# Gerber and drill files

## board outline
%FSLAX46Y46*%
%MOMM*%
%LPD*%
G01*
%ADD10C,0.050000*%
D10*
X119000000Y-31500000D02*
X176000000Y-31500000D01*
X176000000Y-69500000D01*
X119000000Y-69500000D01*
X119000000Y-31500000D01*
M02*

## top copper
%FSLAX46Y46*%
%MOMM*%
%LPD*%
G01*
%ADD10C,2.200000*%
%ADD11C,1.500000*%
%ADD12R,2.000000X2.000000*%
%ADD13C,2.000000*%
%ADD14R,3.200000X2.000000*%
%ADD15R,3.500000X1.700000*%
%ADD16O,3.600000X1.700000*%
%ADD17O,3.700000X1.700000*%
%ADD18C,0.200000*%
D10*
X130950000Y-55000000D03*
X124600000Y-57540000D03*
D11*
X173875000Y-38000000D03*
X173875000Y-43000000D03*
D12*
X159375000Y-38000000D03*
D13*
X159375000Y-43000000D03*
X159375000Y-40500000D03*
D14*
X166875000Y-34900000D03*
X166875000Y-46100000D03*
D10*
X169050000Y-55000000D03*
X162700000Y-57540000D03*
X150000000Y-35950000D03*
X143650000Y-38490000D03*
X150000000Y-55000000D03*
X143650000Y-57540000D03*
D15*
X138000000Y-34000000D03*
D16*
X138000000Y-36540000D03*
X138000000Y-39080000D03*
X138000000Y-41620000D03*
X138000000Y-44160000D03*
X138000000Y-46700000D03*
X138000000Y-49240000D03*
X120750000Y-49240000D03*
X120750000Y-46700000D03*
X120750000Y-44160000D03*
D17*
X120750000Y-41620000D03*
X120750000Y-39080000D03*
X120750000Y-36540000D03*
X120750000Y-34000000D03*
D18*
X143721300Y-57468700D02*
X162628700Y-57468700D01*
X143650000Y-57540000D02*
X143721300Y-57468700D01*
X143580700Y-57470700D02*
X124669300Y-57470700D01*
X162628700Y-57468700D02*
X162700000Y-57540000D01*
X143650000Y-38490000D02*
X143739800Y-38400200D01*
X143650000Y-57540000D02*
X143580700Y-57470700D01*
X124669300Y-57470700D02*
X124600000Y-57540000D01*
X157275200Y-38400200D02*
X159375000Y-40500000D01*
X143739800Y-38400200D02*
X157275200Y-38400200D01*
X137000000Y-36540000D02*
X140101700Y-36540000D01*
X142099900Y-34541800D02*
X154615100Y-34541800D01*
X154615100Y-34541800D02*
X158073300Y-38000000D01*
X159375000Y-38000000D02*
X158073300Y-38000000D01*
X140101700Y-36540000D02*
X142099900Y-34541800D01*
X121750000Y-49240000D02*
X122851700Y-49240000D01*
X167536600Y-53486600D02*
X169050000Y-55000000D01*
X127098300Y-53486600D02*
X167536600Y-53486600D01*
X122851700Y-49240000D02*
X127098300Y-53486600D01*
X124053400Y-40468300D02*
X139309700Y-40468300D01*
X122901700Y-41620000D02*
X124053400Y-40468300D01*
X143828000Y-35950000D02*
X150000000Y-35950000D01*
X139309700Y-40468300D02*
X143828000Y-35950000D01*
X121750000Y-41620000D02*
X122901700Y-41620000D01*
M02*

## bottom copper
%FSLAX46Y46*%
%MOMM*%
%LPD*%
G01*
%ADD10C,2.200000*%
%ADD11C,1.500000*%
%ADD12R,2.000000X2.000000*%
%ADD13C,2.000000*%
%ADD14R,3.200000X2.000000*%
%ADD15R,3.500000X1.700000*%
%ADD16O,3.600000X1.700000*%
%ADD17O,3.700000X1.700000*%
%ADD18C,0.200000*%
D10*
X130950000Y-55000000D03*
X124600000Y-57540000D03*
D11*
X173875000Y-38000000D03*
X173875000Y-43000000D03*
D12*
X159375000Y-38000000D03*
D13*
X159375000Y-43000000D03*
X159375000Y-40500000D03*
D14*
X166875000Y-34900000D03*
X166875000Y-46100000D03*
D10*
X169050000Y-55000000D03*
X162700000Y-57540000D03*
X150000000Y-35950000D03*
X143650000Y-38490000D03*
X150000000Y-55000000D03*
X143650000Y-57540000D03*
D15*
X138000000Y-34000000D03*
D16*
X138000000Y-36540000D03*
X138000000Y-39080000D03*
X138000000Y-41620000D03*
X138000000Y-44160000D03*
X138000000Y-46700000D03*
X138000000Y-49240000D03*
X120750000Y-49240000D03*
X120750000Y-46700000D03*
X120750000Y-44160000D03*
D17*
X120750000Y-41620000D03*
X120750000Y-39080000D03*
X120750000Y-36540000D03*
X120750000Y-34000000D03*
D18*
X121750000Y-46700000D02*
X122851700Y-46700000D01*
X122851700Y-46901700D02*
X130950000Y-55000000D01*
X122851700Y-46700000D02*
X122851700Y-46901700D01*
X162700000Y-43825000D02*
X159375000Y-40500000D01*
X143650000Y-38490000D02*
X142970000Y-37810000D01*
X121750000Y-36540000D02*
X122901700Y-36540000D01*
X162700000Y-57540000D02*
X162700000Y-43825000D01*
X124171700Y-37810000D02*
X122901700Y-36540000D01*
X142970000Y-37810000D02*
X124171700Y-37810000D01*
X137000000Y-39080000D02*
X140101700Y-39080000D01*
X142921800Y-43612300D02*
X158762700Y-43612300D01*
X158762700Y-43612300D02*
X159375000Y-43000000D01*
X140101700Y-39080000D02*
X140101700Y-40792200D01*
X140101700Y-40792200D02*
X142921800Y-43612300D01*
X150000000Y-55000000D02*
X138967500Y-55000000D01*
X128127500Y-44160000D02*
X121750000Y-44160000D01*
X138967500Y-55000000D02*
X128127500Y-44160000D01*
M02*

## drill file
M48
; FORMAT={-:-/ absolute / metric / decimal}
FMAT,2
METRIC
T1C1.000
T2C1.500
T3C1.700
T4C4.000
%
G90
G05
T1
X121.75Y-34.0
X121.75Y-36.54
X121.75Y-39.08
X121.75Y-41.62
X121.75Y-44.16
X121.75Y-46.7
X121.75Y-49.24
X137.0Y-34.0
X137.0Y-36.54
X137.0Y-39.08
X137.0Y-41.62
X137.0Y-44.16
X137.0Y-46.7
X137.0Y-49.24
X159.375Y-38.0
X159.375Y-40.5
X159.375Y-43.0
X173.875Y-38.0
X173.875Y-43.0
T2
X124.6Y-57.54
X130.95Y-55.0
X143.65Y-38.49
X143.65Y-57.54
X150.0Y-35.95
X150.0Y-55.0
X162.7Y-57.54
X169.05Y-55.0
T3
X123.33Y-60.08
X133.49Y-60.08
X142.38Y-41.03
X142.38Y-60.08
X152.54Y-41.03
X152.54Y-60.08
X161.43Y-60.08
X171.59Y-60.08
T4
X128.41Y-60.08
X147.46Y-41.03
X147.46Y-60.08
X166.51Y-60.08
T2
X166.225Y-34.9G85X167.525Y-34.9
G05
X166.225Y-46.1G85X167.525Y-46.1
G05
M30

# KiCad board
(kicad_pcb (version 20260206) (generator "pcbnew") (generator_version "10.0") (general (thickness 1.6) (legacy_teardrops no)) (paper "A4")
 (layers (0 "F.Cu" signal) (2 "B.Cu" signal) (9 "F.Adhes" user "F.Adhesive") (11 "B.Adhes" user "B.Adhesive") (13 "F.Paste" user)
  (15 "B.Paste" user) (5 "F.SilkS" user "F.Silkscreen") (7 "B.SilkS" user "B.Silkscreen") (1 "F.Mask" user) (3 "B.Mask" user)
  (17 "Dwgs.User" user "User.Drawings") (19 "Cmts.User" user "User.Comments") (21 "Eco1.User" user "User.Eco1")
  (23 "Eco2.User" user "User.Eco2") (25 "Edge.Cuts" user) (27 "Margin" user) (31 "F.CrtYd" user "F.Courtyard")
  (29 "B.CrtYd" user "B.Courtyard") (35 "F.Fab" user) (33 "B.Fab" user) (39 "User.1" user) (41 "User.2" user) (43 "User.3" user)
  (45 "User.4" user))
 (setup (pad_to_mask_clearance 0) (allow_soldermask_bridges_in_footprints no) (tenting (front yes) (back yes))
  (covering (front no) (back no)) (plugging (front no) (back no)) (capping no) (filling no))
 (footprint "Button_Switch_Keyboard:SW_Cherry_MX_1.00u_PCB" (layer "F.Cu") (at 130.95 55)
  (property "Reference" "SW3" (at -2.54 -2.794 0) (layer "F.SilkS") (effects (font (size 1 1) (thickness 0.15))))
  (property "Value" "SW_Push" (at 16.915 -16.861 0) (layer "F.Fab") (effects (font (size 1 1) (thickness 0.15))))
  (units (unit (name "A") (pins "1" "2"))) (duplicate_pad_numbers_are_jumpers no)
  (pad "" np_thru_hole circle (at -7.62 5.08) (size 1.7 1.7) (drill 1.7) (layers "*.Cu" "*.Mask"))
  (pad "" np_thru_hole circle (at -2.54 5.08) (size 4 4) (drill 4) (layers "*.Cu" "*.Mask"))
  (pad "" np_thru_hole circle (at 2.54 5.08) (size 1.7 1.7) (drill 1.7) (layers "*.Cu" "*.Mask"))
  (pad "1" thru_hole circle (at 0 0) (size 2.2 2.2) (drill 1.5) (layers "*.Cu" "*.Mask") (remove_unused_layers no)
   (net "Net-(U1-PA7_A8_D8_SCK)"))
  (pad "2" thru_hole circle (at -6.35 2.54) (size 2.2 2.2) (drill 1.5) (layers "*.Cu" "*.Mask") (remove_unused_layers no) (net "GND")))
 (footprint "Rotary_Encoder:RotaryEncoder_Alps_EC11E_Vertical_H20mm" (layer "F.Cu") (at 159.375 38)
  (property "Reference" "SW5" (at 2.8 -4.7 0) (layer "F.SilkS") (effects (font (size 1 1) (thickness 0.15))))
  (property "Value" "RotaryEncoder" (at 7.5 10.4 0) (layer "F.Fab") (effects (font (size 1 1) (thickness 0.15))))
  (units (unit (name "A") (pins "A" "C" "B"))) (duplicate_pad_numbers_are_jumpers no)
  (pad "" thru_hole circle (at 14.5 0) (size 1.5 1.5) (drill 1) (layers "*.Cu" "*.Mask") (remove_unused_layers no))
  (pad "" thru_hole circle (at 14.5 5) (size 1.5 1.5) (drill 1) (layers "*.Cu" "*.Mask") (remove_unused_layers no))
  (pad "A" thru_hole rect (at 0 0) (size 2 2) (drill 1) (layers "*.Cu" "*.Mask") (remove_unused_layers no) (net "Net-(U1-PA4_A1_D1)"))
  (pad "B" thru_hole circle (at 0 5) (size 2 2) (drill 1) (layers "*.Cu" "*.Mask") (remove_unused_layers no) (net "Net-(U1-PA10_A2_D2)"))
  (pad "C" thru_hole circle (at 0 2.5) (size 2 2) (drill 1) (layers "*.Cu" "*.Mask") (remove_unused_layers no) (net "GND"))
  (pad "MP" thru_hole rect (at 7.5 -3.1) (size 3.2 2) (drill oval 2.8 1.5) (layers "*.Cu" "*.Mask") (remove_unused_layers no))
  (pad "MP" thru_hole rect (at 7.5 8.1) (size 3.2 2) (drill oval 2.8 1.5) (layers "*.Cu" "*.Mask") (remove_unused_layers no)))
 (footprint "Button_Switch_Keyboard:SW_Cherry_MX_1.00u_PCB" (layer "F.Cu") (at 169.05 55)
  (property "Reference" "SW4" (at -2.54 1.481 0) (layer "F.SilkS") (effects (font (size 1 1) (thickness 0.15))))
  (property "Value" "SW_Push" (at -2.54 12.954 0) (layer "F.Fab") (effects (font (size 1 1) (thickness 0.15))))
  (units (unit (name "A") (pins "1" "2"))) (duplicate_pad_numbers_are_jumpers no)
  (pad "" np_thru_hole circle (at -7.62 5.08) (size 1.7 1.7) (drill 1.7) (layers "*.Cu" "*.Mask"))
  (pad "" np_thru_hole circle (at -2.54 5.08) (size 4 4) (drill 4) (layers "*.Cu" "*.Mask"))
  (pad "" np_thru_hole circle (at 2.54 5.08) (size 1.7 1.7) (drill 1.7) (layers "*.Cu" "*.Mask"))
  (pad "1" thru_hole circle (at 0 0) (size 2.2 2.2) (drill 1.5) (layers "*.Cu" "*.Mask") (remove_unused_layers no)
   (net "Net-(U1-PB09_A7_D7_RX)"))
  (pad "2" thru_hole circle (at -6.35 2.54) (size 2.2 2.2) (drill 1.5) (layers "*.Cu" "*.Mask") (remove_unused_layers no) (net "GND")))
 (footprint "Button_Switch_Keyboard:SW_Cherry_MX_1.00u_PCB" (layer "F.Cu") (at 150 35.95)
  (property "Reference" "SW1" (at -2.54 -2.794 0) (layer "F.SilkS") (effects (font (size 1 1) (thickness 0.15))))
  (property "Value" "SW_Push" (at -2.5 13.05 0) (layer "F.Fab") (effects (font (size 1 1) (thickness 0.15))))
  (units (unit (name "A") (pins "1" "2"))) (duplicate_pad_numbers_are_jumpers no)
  (pad "" np_thru_hole circle (at -7.62 5.08) (size 1.7 1.7) (drill 1.7) (layers "*.Cu" "*.Mask"))
  (pad "" np_thru_hole circle (at -2.54 5.08) (size 4 4) (drill 4) (layers "*.Cu" "*.Mask"))
  (pad "" np_thru_hole circle (at 2.54 5.08) (size 1.7 1.7) (drill 1.7) (layers "*.Cu" "*.Mask"))
  (pad "1" thru_hole circle (at 0 0) (size 2.2 2.2) (drill 1.5) (layers "*.Cu" "*.Mask") (remove_unused_layers no)
   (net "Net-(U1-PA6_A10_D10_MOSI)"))
  (pad "2" thru_hole circle (at -6.35 2.54) (size 2.2 2.2) (drill 1.5) (layers "*.Cu" "*.Mask") (remove_unused_layers no) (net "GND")))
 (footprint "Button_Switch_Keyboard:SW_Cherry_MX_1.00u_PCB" (layer "F.Cu") (at 150 55)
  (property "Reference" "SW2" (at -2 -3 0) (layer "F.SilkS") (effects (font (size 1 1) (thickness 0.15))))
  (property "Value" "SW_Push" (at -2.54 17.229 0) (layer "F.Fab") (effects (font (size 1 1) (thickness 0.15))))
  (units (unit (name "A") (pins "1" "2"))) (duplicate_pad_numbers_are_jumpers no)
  (pad "" np_thru_hole circle (at -7.62 5.08) (size 1.7 1.7) (drill 1.7) (layers "*.Cu" "*.Mask"))
  (pad "" np_thru_hole circle (at -2.54 5.08) (size 4 4) (drill 4) (layers "*.Cu" "*.Mask"))
  (pad "" np_thru_hole circle (at 2.54 5.08) (size 1.7 1.7) (drill 1.7) (layers "*.Cu" "*.Mask"))
  (pad "1" thru_hole circle (at 0 0) (size 2.2 2.2) (drill 1.5) (layers "*.Cu" "*.Mask") (remove_unused_layers no)
   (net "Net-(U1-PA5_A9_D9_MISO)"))
  (pad "2" thru_hole circle (at -6.35 2.54) (size 2.2 2.2) (drill 1.5) (layers "*.Cu" "*.Mask") (remove_unused_layers no) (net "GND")))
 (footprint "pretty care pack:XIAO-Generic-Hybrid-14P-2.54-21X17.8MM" (layer "B.Cu") (at 129.375 41.62 180)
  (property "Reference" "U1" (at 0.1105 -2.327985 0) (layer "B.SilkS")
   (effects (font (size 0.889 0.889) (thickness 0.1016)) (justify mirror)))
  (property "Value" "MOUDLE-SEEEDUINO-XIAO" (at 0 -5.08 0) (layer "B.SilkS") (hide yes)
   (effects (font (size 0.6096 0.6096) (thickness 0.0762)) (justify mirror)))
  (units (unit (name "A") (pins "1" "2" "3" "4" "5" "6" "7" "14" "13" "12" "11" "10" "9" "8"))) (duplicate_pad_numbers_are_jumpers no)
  (pad "1" thru_hole rect (at -7.625 7.62 180) (size 3.5 1.7) (drill 1 (offset -1 0)) (layers "*.Cu" "*.Mask") (remove_unused_layers no)
   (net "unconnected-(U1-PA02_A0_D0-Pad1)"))
  (pad "2" thru_hole oval (at -7.625 5.08 180) (size 3.6 1.7) (drill 1 (offset -1 0)) (layers "*.Cu" "*.Mask") (remove_unused_layers no)
   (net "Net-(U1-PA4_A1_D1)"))
  (pad "3" thru_hole oval (at -7.625 2.54 180) (size 3.6 1.7) (drill 1 (offset -1 0)) (layers "*.Cu" "*.Mask") (remove_unused_layers no)
   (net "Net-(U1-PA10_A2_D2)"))
  (pad "4" thru_hole oval (at -7.625 0 180) (size 3.6 1.7) (drill 1 (offset -1 0)) (layers "*.Cu" "*.Mask") (remove_unused_layers no)
   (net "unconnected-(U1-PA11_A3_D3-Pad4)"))
  (pad "5" thru_hole oval (at -7.625 -2.54 180) (size 3.6 1.7) (drill 1 (offset -1 0)) (layers "*.Cu" "*.Mask") (remove_unused_layers no)
   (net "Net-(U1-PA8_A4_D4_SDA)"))
  (pad "6" thru_hole oval (at -7.625 -5.08) (size 3.6 1.7) (drill 1 (offset 1 0)) (layers "*.Cu" "*.Mask") (remove_unused_layers no)
   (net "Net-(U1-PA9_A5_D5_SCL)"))
  (pad "7" thru_hole oval (at -7.625 -7.62 180) (size 3.6 1.7) (drill 1 (offset -1 0)) (layers "*.Cu" "*.Mask") (remove_unused_layers no)
   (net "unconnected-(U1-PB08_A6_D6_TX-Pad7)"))
  (pad "8" thru_hole oval (at 7.625 -7.62 180) (size 3.6 1.7) (drill 1 (offset 1 0)) (layers "*.Cu" "*.Mask") (remove_unused_layers no)
   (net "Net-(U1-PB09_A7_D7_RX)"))
  (pad "9" thru_hole oval (at 7.625 -5.08 180) (size 3.6 1.7) (drill 1 (offset 1 0)) (layers "*.Cu" "*.Mask") (remove_unused_layers no)
   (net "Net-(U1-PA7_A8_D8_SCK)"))
  (pad "10" thru_hole oval (at 7.625 -2.54 180) (size 3.6 1.7) (drill 1 (offset 1 0)) (layers "*.Cu" "*.Mask") (remove_unused_layers no)
   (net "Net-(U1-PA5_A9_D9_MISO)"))
  (pad "11" thru_hole oval (at 7.625 0 180) (size 3.7 1.7) (drill 1 (offset 1 0)) (layers "*.Cu" "*.Mask") (remove_unused_layers no)
   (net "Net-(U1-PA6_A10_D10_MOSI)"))
  (pad "12" thru_hole oval (at 7.625 2.54 180) (size 3.7 1.7) (drill 1 (offset 1 0)) (layers "*.Cu" "*.Mask") (remove_unused_layers no)
   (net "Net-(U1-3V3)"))
  (pad "13" thru_hole oval (at 7.625 5.08 180) (size 3.7 1.7) (drill 1 (offset 1 0)) (layers "*.Cu" "*.Mask") (remove_unused_layers no)
   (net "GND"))
  (pad "14" thru_hole oval (at 7.625 7.62 180) (size 3.7 1.7) (drill 1 (offset 1 0)) (layers "*.Cu" "*.Mask") (remove_unused_layers no)
   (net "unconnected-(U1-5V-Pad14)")))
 (gr_rect (start 119 31.5) (end 176 69.5) (stroke (width 0.05) (type default)) (fill no) (layer "Edge.Cuts"))
 (segment (start 121.75 46.7) (end 122.8517 46.7) (width 0.2) (layer "B.Cu") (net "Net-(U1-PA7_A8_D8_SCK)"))
 (segment (start 122.8517 46.9017) (end 130.95 55) (width 0.2) (layer "B.Cu") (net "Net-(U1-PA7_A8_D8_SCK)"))
 (segment (start 122.8517 46.7) (end 122.8517 46.9017) (width 0.2) (layer "B.Cu") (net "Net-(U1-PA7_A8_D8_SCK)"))
 (segment (start 143.7213 57.4687) (end 162.6287 57.4687) (width 0.2) (layer "F.Cu") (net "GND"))
 (segment (start 143.65 57.54) (end 143.7213 57.4687) (width 0.2) (layer "F.Cu") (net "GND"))
 (segment (start 143.5807 57.4707) (end 124.6693 57.4707) (width 0.2) (layer "F.Cu") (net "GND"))
 (segment (start 162.6287 57.4687) (end 162.7 57.54) (width 0.2) (layer "F.Cu") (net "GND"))
 (segment (start 143.65 38.49) (end 143.7398 38.4002) (width 0.2) (layer "F.Cu") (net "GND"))
 (segment (start 143.65 57.54) (end 143.5807 57.4707) (width 0.2) (layer "F.Cu") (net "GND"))
 (segment (start 124.6693 57.4707) (end 124.6 57.54) (width 0.2) (layer "F.Cu") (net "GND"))
 (segment (start 157.2752 38.4002) (end 159.375 40.5) (width 0.2) (layer "F.Cu") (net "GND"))
 (segment (start 143.7398 38.4002) (end 157.2752 38.4002) (width 0.2) (layer "F.Cu") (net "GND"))
 (segment (start 162.7 43.825) (end 159.375 40.5) (width 0.2) (layer "B.Cu") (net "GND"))
 (segment (start 143.65 38.49) (end 142.97 37.81) (width 0.2) (layer "B.Cu") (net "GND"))
 (segment (start 121.75 36.54) (end 122.9017 36.54) (width 0.2) (layer "B.Cu") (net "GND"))
 (segment (start 162.7 57.54) (end 162.7 43.825) (width 0.2) (layer "B.Cu") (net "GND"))
 (segment (start 124.1717 37.81) (end 122.9017 36.54) (width 0.2) (layer "B.Cu") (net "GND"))
 (segment (start 142.97 37.81) (end 124.1717 37.81) (width 0.2) (layer "B.Cu") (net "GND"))
 (segment (start 137 36.54) (end 140.1017 36.54) (width 0.2) (layer "F.Cu") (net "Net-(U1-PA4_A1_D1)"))
 (segment (start 142.0999 34.5418) (end 154.6151 34.5418) (width 0.2) (layer "F.Cu") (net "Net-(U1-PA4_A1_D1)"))
 (segment (start 154.6151 34.5418) (end 158.0733 38) (width 0.2) (layer "F.Cu") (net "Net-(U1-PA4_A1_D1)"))
 (segment (start 159.375 38) (end 158.0733 38) (width 0.2) (layer "F.Cu") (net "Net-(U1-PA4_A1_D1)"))
 (segment (start 140.1017 36.54) (end 142.0999 34.5418) (width 0.2) (layer "F.Cu") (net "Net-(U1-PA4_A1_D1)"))
 (segment (start 137 39.08) (end 140.1017 39.08) (width 0.2) (layer "B.Cu") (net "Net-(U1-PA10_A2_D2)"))
 (segment (start 142.9218 43.6123) (end 158.7627 43.6123) (width 0.2) (layer "B.Cu") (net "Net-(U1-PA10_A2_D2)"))
 (segment (start 158.7627 43.6123) (end 159.375 43) (width 0.2) (layer "B.Cu") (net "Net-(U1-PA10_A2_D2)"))
 (segment (start 140.1017 39.08) (end 140.1017 40.7922) (width 0.2) (layer "B.Cu") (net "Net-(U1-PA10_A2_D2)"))
 (segment (start 140.1017 40.7922) (end 142.9218 43.6123) (width 0.2) (layer "B.Cu") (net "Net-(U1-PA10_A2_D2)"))
 (segment (start 121.75 49.24) (end 122.8517 49.24) (width 0.2) (layer "F.Cu") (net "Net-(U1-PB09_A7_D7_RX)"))
 (segment (start 167.5366 53.4866) (end 169.05 55) (width 0.2) (layer "F.Cu") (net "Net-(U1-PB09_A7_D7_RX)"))
 (segment (start 127.0983 53.4866) (end 167.5366 53.4866) (width 0.2) (layer "F.Cu") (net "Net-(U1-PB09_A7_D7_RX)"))
 (segment (start 122.8517 49.24) (end 127.0983 53.4866) (width 0.2) (layer "F.Cu") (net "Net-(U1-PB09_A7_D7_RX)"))
 (segment (start 124.0534 40.4683) (end 139.3097 40.4683) (width 0.2) (layer "F.Cu") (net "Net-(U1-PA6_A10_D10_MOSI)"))
 (segment (start 122.9017 41.62) (end 124.0534 40.4683) (width 0.2) (layer "F.Cu") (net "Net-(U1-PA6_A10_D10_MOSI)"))
 (segment (start 143.828 35.95) (end 150 35.95) (width 0.2) (layer "F.Cu") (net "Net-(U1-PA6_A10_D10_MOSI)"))
 (segment (start 139.3097 40.4683) (end 143.828 35.95) (width 0.2) (layer "F.Cu") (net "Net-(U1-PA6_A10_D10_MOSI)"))
 (segment (start 121.75 41.62) (end 122.9017 41.62) (width 0.2) (layer "F.Cu") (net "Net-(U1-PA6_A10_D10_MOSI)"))
 (segment (start 150 55) (end 138.9675 55) (width 0.2) (layer "B.Cu") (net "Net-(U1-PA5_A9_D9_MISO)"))
 (segment (start 128.1275 44.16) (end 121.75 44.16) (width 0.2) (layer "B.Cu") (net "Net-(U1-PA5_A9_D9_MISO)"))
 (segment (start 138.9675 55) (end 128.1275 44.16) (width 0.2) (layer "B.Cu") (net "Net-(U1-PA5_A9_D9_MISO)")))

